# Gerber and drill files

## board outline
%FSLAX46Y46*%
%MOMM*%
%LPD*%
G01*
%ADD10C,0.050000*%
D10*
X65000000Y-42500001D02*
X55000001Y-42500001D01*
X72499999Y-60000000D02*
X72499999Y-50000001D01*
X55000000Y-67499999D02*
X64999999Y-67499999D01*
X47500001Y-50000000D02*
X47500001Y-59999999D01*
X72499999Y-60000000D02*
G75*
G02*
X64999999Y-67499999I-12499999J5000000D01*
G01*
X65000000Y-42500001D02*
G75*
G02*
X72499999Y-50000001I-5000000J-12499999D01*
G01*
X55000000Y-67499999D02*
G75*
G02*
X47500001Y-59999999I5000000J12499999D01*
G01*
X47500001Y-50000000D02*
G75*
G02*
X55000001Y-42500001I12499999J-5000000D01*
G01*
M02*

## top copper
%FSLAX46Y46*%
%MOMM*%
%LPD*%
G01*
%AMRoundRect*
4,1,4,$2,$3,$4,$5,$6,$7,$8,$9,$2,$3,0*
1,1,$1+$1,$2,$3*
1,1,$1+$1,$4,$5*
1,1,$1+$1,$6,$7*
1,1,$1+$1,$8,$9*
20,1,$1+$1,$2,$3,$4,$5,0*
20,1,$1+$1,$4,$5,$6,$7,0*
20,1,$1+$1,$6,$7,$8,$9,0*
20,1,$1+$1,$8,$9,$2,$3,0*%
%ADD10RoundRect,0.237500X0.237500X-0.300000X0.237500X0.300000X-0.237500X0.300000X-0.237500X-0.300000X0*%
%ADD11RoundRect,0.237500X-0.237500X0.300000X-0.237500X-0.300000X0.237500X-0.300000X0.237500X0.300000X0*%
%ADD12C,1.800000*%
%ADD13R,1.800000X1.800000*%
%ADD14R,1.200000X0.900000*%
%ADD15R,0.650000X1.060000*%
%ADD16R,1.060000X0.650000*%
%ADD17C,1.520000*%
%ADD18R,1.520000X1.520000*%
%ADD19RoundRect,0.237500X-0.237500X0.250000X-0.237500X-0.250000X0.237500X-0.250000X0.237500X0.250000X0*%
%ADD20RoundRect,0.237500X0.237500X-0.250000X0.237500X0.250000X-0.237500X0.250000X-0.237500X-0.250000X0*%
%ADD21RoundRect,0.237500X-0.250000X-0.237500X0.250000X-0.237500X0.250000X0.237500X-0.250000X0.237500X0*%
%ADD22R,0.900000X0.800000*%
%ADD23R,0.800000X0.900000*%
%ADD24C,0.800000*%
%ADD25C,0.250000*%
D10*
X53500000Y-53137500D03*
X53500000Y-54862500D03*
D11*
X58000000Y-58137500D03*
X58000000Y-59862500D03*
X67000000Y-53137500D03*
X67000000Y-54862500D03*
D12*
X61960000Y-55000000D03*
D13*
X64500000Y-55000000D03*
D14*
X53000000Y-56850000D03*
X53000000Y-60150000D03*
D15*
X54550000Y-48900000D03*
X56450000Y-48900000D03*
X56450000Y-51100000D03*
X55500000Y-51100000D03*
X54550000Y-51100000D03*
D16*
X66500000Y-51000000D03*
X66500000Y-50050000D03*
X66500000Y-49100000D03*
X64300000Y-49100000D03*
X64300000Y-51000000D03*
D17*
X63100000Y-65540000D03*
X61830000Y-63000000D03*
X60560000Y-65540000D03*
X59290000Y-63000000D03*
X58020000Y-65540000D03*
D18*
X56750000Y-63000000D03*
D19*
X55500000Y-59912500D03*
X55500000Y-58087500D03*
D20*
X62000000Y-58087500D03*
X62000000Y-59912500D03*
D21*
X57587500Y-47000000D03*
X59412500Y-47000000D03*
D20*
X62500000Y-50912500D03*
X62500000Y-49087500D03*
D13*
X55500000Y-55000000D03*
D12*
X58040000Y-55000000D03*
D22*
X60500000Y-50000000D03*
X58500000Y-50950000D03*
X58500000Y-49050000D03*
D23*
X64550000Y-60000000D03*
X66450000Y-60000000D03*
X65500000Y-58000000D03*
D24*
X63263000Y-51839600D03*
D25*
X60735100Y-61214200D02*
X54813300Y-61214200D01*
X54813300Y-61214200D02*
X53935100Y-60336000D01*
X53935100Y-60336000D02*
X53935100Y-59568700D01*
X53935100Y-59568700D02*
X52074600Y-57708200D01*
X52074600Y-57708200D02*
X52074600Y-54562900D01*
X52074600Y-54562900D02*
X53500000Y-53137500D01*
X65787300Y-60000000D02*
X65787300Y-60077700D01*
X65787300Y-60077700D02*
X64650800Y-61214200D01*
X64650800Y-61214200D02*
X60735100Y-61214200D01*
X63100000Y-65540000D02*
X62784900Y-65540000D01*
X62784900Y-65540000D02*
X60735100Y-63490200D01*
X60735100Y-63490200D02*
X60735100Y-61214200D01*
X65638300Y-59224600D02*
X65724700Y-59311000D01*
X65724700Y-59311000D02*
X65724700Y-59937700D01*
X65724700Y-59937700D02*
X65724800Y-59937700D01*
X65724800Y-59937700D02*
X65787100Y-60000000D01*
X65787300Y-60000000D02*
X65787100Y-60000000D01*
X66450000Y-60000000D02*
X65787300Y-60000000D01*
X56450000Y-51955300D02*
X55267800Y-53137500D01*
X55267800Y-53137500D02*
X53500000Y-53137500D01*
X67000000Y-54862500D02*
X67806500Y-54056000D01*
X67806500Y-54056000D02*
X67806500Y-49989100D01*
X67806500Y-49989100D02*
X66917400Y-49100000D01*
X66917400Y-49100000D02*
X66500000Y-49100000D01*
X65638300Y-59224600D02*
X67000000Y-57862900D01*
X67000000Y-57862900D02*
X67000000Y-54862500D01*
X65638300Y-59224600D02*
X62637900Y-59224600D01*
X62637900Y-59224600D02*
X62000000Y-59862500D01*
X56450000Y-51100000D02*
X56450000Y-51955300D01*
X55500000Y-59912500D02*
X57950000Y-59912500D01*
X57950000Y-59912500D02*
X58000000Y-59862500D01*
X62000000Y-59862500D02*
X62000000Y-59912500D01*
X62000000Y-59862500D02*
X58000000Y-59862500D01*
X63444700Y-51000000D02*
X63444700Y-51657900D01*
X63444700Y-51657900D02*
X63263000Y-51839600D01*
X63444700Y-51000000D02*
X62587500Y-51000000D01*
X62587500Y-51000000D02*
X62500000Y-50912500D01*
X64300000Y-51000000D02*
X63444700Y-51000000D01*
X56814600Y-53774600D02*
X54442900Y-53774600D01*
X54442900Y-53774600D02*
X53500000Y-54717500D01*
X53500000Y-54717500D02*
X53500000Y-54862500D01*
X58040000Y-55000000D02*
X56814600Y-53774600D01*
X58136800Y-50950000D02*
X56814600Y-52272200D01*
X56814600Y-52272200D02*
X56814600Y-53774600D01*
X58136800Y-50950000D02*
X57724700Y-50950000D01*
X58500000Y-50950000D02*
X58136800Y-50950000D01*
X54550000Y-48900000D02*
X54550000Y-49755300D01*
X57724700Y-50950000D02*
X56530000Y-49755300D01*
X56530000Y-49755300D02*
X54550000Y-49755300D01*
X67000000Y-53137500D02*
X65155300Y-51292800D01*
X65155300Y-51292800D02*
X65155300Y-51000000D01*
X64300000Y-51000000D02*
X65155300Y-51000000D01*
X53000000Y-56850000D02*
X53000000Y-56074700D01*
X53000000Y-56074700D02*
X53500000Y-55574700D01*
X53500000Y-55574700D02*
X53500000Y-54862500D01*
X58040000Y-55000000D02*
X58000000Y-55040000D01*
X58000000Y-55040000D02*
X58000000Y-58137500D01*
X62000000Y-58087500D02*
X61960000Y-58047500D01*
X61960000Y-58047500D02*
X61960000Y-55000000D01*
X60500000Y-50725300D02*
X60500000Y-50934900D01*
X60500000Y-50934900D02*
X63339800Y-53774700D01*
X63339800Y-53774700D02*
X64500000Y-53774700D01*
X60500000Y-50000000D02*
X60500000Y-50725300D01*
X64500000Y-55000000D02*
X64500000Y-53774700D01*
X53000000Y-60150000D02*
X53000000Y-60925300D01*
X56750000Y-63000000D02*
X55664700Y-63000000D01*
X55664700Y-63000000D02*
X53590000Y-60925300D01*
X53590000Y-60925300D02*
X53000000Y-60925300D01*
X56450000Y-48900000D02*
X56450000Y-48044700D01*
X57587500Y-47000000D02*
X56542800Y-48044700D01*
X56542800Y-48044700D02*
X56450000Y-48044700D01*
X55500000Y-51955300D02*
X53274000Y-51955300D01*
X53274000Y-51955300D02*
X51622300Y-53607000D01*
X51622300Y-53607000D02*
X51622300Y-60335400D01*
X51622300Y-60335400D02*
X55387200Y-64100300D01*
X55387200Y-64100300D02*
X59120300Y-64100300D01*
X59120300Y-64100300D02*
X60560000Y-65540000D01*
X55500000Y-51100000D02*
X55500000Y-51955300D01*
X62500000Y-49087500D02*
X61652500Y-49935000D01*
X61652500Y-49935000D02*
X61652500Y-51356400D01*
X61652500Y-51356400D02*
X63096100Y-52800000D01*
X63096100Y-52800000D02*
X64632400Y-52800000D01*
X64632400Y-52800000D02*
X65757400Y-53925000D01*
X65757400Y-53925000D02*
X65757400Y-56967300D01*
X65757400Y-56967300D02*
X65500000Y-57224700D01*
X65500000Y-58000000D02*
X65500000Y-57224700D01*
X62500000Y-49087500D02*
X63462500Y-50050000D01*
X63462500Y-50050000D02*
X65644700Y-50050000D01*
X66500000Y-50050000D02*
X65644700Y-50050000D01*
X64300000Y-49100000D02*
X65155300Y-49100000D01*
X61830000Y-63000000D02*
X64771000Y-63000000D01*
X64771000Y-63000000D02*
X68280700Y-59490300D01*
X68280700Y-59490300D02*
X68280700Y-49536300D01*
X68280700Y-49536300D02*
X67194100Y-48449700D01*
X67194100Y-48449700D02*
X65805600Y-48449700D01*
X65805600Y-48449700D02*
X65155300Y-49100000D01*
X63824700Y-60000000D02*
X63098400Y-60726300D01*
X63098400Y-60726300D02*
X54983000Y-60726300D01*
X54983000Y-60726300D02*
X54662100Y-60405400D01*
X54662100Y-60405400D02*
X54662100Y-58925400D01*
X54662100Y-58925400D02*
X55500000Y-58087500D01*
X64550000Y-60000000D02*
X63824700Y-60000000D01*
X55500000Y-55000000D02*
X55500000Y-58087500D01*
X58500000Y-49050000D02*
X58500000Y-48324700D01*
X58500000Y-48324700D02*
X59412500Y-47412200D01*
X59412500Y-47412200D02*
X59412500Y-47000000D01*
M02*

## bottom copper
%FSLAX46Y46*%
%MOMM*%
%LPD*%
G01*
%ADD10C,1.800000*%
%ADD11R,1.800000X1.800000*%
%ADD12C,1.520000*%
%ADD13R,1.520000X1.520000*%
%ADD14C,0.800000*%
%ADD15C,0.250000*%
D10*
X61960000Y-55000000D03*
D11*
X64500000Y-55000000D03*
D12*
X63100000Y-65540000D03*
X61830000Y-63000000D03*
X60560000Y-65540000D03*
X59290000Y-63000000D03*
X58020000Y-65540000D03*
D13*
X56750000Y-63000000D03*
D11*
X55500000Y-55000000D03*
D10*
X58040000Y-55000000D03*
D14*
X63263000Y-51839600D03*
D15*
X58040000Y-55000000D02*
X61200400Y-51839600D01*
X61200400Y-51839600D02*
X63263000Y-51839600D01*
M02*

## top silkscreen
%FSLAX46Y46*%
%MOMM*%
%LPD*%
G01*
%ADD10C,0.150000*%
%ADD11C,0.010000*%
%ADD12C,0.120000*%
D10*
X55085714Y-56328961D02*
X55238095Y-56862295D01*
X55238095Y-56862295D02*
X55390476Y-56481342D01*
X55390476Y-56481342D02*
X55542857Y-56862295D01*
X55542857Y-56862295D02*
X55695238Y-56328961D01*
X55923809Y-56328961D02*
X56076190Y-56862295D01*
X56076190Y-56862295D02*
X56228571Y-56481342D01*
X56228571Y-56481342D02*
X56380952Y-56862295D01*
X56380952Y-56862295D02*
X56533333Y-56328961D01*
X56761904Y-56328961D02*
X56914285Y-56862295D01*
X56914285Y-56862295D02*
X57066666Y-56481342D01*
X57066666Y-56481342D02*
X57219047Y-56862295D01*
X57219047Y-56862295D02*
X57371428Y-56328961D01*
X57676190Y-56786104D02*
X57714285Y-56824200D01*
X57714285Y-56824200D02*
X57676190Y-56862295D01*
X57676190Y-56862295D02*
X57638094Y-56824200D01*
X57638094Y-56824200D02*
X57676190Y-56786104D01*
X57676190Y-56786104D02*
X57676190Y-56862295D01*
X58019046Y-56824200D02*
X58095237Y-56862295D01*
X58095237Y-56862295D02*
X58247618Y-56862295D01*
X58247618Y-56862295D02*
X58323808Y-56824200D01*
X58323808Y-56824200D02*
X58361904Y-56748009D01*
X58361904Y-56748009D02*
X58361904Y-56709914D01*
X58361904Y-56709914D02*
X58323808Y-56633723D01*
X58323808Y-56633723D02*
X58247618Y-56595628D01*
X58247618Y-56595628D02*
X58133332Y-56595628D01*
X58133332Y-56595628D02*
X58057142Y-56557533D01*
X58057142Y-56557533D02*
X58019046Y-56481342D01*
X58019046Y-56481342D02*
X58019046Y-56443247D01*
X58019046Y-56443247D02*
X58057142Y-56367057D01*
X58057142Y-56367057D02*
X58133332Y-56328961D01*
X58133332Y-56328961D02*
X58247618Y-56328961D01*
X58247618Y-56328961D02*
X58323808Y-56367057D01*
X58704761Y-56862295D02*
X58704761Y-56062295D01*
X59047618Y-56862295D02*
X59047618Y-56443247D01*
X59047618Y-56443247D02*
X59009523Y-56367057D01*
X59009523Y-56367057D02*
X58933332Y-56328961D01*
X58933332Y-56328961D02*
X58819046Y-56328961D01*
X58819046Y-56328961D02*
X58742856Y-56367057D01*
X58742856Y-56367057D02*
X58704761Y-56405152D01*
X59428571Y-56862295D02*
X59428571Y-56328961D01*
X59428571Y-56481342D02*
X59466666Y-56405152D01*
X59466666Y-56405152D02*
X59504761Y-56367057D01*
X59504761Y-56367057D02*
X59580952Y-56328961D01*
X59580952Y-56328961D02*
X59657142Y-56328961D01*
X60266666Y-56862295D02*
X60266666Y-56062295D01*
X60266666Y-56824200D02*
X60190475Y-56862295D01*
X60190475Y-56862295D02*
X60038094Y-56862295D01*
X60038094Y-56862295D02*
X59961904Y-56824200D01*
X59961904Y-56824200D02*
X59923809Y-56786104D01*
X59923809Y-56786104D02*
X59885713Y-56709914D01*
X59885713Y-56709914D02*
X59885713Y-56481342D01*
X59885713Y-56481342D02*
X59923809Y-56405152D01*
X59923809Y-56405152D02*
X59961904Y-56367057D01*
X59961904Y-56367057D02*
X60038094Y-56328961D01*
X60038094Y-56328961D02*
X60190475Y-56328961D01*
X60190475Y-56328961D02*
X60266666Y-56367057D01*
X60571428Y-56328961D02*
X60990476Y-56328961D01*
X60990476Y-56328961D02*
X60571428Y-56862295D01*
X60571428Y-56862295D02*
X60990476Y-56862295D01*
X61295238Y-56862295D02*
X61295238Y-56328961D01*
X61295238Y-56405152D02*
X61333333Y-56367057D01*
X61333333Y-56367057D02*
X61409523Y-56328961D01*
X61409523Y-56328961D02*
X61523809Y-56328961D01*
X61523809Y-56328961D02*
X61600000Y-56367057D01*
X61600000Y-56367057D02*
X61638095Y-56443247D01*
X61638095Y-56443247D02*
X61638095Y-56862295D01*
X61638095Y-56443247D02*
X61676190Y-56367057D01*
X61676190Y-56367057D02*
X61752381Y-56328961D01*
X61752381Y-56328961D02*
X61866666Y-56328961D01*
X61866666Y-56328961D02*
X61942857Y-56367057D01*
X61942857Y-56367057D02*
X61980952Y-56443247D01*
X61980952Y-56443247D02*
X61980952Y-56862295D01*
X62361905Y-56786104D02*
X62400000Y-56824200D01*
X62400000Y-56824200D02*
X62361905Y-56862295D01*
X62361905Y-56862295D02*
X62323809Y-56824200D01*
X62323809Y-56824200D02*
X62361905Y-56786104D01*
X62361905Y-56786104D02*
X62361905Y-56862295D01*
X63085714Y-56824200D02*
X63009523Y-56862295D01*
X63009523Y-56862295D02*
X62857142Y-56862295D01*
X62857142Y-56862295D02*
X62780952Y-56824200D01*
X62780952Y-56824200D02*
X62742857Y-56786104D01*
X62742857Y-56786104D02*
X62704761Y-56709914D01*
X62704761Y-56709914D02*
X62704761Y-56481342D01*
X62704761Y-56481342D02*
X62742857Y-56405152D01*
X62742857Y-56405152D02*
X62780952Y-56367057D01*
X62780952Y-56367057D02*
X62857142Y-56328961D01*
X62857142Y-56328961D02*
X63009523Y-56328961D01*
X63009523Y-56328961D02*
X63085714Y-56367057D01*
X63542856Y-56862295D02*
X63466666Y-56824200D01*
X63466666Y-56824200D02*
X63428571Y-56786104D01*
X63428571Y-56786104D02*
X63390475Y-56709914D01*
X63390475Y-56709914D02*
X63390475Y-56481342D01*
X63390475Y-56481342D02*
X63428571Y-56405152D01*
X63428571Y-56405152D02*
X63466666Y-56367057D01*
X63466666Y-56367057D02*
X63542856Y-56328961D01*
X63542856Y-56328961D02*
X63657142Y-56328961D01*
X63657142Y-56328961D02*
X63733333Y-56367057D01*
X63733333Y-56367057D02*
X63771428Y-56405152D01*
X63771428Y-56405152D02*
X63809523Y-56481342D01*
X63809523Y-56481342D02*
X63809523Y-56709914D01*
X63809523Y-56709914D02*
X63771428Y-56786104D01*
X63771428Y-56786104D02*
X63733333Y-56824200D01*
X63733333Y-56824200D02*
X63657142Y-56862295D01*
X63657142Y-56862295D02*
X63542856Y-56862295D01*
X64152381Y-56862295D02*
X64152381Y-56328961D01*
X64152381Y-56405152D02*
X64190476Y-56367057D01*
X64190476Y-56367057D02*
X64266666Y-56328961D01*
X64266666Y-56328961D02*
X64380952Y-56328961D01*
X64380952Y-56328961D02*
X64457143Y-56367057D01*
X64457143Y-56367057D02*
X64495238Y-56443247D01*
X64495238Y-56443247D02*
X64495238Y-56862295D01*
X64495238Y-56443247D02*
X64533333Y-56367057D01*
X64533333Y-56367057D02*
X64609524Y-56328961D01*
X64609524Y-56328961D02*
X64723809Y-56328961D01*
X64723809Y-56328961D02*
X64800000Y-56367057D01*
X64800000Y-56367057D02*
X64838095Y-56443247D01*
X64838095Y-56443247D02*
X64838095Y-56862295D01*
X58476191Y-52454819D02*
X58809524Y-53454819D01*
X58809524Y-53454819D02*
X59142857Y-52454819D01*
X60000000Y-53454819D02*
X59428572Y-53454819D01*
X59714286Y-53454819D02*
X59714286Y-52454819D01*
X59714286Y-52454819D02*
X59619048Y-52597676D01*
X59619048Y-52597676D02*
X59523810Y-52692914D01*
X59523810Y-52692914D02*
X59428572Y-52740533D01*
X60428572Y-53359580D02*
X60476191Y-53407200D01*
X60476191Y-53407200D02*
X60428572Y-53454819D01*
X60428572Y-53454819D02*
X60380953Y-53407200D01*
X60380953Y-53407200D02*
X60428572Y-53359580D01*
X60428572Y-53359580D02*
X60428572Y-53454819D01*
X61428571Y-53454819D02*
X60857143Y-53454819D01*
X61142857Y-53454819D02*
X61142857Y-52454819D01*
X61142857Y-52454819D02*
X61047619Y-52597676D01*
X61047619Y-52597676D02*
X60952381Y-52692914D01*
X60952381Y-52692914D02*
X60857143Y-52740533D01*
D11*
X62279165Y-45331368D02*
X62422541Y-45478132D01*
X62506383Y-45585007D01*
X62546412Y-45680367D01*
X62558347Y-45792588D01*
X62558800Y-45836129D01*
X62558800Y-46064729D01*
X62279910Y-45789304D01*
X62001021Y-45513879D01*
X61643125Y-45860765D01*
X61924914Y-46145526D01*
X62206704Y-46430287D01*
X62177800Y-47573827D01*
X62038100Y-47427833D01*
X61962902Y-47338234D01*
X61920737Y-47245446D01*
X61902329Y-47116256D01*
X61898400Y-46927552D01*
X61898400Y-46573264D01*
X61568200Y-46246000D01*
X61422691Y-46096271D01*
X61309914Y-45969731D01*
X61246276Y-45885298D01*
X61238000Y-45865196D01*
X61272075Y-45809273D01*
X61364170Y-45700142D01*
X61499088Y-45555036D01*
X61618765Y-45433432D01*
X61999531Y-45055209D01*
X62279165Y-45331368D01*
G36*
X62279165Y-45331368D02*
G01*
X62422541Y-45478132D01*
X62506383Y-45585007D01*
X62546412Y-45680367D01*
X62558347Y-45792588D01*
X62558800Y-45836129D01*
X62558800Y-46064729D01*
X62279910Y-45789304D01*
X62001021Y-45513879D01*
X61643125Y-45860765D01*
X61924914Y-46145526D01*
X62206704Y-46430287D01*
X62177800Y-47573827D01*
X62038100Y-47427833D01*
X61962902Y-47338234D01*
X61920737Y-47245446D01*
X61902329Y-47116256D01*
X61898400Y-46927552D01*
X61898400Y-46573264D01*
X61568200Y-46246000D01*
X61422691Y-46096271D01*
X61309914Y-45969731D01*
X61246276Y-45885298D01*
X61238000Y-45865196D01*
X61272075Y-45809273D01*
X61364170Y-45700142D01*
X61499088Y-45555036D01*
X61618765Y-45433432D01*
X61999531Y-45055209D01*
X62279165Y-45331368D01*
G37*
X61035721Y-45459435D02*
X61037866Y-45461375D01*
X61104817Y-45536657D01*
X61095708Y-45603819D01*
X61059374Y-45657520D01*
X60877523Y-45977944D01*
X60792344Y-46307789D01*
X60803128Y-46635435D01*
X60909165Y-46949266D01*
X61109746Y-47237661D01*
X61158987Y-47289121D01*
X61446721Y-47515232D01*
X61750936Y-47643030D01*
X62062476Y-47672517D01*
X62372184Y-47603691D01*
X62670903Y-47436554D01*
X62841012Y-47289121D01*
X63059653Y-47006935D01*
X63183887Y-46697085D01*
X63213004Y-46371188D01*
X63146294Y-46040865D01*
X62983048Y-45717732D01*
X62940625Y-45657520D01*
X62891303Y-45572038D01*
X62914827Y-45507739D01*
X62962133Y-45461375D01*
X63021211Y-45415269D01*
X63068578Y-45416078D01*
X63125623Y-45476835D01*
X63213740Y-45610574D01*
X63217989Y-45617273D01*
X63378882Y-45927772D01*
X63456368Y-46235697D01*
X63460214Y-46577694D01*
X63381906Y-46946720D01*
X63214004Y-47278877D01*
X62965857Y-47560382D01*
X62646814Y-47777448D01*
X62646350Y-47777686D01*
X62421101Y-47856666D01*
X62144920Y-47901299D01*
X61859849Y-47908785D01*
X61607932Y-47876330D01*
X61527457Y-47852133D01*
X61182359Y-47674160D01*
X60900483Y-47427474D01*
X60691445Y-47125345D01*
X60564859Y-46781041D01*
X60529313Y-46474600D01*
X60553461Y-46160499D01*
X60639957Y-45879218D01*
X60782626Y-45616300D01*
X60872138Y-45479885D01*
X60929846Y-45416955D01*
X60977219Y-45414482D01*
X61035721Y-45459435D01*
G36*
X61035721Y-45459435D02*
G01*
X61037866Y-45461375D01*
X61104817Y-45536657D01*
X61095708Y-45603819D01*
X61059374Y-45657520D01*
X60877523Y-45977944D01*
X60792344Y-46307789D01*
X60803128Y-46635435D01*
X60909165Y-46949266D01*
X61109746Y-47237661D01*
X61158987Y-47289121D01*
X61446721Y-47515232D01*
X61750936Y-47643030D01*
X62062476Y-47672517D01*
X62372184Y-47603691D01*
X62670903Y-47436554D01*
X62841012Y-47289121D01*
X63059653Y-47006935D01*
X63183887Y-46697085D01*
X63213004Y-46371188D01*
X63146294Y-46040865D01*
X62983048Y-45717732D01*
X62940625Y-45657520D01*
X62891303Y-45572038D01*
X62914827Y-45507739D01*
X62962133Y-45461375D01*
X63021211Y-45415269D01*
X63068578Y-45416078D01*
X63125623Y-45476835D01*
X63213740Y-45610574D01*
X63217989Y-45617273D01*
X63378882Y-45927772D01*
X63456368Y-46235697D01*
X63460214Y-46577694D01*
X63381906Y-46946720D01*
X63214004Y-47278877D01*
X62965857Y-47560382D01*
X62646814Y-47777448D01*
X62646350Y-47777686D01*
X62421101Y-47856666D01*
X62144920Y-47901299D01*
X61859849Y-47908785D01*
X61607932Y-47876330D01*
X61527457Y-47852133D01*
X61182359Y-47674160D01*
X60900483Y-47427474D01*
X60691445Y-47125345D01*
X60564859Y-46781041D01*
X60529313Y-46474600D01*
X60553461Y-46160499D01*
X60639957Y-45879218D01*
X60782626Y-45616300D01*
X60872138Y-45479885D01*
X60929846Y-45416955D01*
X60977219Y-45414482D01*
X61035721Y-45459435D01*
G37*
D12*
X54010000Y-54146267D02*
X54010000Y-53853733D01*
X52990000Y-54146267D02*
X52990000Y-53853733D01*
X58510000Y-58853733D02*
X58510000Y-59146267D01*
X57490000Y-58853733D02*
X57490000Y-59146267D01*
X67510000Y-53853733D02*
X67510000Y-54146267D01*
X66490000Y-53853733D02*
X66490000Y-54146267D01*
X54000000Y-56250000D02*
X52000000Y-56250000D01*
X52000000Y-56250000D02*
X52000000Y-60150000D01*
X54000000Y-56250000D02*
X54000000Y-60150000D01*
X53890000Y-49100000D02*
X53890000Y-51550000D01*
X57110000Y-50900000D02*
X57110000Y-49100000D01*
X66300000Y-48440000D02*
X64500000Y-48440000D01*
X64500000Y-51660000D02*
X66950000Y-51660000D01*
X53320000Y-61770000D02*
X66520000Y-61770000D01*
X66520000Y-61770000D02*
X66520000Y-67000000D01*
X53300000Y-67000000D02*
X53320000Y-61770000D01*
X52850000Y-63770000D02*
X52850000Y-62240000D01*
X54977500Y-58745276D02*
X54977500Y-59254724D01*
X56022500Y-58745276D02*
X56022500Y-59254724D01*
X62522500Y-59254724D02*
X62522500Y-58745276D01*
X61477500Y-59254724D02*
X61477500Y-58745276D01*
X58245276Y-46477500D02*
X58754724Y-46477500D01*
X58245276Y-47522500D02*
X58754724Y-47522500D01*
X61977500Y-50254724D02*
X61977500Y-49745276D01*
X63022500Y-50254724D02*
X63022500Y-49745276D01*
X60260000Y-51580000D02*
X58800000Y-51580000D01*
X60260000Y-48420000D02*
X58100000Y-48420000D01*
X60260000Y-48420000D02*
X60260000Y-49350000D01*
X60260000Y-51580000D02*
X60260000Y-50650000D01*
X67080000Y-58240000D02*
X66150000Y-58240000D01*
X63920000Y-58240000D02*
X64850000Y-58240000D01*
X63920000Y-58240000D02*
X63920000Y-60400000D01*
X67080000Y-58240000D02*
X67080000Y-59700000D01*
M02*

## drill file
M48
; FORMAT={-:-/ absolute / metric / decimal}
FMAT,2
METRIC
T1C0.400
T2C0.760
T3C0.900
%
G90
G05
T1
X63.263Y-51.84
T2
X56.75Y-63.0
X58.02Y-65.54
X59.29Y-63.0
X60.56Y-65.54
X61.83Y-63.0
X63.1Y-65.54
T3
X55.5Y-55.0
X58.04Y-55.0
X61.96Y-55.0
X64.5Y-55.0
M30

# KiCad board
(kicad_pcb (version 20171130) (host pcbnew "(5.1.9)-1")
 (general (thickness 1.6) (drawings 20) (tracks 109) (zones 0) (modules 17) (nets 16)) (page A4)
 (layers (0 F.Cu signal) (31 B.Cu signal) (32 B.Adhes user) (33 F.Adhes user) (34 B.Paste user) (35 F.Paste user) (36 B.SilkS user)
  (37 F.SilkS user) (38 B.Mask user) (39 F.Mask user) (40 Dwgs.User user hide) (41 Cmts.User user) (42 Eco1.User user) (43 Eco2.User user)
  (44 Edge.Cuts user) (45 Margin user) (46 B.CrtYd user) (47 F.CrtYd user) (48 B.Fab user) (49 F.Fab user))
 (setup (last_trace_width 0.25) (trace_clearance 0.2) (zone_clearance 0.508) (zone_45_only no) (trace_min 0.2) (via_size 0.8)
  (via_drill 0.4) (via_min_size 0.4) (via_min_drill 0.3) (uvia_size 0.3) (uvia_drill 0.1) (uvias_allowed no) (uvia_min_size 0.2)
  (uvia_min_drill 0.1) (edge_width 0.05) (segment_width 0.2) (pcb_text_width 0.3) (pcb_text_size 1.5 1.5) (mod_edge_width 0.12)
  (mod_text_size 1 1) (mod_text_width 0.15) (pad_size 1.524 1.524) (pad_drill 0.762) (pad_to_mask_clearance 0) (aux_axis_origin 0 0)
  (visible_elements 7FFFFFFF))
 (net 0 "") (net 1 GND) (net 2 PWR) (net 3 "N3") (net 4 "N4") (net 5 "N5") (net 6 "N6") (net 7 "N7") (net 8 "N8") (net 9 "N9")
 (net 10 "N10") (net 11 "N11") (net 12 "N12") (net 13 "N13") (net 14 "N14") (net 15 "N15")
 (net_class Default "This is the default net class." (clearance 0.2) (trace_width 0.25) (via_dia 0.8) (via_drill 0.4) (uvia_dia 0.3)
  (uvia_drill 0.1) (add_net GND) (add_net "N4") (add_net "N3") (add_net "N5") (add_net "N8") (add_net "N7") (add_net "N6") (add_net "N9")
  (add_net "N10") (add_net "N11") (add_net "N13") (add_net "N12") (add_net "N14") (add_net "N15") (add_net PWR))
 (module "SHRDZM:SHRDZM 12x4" (layer B.Cu) (at 60.5 50 180)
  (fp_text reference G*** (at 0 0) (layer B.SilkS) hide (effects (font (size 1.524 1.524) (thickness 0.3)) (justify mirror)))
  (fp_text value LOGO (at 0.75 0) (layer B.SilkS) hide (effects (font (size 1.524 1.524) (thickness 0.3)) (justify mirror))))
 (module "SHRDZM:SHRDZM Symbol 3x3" (layer F.Cu) (at 62 46.5)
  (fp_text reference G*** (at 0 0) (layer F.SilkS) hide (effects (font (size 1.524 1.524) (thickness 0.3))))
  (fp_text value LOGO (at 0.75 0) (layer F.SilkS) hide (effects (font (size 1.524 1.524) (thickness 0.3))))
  (fp_poly
   (pts (xy 0.279165 -1.168632) (xy 0.422541 -1.021868) (xy 0.506383 -0.914993) (xy 0.546412 -0.819633) (xy 0.558347 -0.707412)
    (xy 0.5588 -0.663871) (xy 0.5588 -0.435271) (xy 0.27991 -0.710696) (xy 0.001021 -0.986121) (xy -0.356875 -0.639235)
    (xy -0.075086 -0.354474) (xy 0.206704 -0.069713) (xy 0.1778 1.073827) (xy 0.0381 0.927833) (xy -0.037098 0.838234)
    (xy -0.079263 0.745446) (xy -0.097671 0.616256) (xy -0.1016 0.427552) (xy -0.1016 0.073264) (xy -0.4318 -0.254) (xy -0.577309 -0.403729)
    (xy -0.690086 -0.530269) (xy -0.753724 -0.614702) (xy -0.762 -0.634804) (xy -0.727925 -0.690727) (xy -0.63583 -0.799858)
    (xy -0.500912 -0.944964) (xy -0.381235 -1.066568) (xy -0.000469 -1.444791) (xy 0.279165 -1.168632))
   (layer F.SilkS) (width 0.01))
  (fp_poly
   (pts (xy -0.964279 -1.040565) (xy -0.962134 -1.038625) (xy -0.895183 -0.963343) (xy -0.904292 -0.896181) (xy -0.940626 -0.84248)
    (xy -1.122477 -0.522056) (xy -1.207656 -0.192211) (xy -1.196872 0.135435) (xy -1.090835 0.449266) (xy -0.890254 0.737661)
    (xy -0.841013 0.789121) (xy -0.553279 1.015232) (xy -0.249064 1.14303) (xy 0.062476 1.172517) (xy 0.372184 1.103691)
    (xy 0.670903 0.936554) (xy 0.841012 0.789121) (xy 1.059653 0.506935) (xy 1.183887 0.197085) (xy 1.213004 -0.128812)
    (xy 1.146294 -0.459135) (xy 0.983048 -0.782268) (xy 0.940625 -0.84248) (xy 0.891303 -0.927962) (xy 0.914827 -0.992261)
    (xy 0.962133 -1.038625) (xy 1.021211 -1.084731) (xy 1.068578 -1.083922) (xy 1.125623 -1.023165) (xy 1.21374 -0.889426)
    (xy 1.217989 -0.882727) (xy 1.378882 -0.572228) (xy 1.456368 -0.264303) (xy 1.460214 0.077694) (xy 1.381906 0.44672)
    (xy 1.214004 0.778877) (xy 0.965857 1.060382) (xy 0.646814 1.277448) (xy 0.64635 1.277686) (xy 0.421101 1.356666) (xy 0.14492 1.401299)
    (xy -0.140151 1.408785) (xy -0.392068 1.37633) (xy -0.472543 1.352133) (xy -0.817641 1.17416) (xy -1.099517 0.927474)
    (xy -1.308555 0.625345) (xy -1.435141 0.281041) (xy -1.470687 -0.0254) (xy -1.446539 -0.339501) (xy -1.360043 -0.620782)
    (xy -1.217374 -0.8837) (xy -1.127862 -1.020115) (xy -1.070154 -1.083045) (xy -1.022781 -1.085518) (xy -0.964279 -1.040565))
   (layer F.SilkS) (width 0.01)))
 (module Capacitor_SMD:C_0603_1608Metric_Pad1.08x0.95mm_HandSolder (layer F.Cu) (at 53.5 54 90)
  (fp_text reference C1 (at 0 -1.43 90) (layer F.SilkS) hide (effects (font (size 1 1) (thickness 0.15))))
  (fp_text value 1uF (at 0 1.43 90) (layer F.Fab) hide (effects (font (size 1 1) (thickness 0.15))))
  (fp_line (start -0.146267 0.51) (end 0.146267 0.51) (layer F.SilkS) (width 0.12))
  (fp_line (start -0.146267 -0.51) (end 0.146267 -0.51) (layer F.SilkS) (width 0.12))
  (pad 2 smd roundrect (at 0.8625 0 90) (size 1.075 0.95) (layers F.Cu F.Paste F.Mask) (roundrect_rratio 0.25) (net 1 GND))
  (pad 1 smd roundrect (at -0.8625 0 90) (size 1.075 0.95) (layers F.Cu F.Paste F.Mask) (roundrect_rratio 0.25) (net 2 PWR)))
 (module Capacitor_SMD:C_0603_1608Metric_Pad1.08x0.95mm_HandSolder (layer F.Cu) (at 58 59 270)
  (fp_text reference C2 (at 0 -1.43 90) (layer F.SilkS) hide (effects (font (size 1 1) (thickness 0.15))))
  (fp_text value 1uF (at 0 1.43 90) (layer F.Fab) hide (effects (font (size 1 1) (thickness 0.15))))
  (fp_line (start -0.146267 -0.51) (end 0.146267 -0.51) (layer F.SilkS) (width 0.12))
  (fp_line (start -0.146267 0.51) (end 0.146267 0.51) (layer F.SilkS) (width 0.12))
  (pad 1 smd roundrect (at -0.8625 0 270) (size 1.075 0.95) (layers F.Cu F.Paste F.Mask) (roundrect_rratio 0.25) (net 2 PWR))
  (pad 2 smd roundrect (at 0.8625 0 270) (size 1.075 0.95) (layers F.Cu F.Paste F.Mask) (roundrect_rratio 0.25) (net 1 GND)))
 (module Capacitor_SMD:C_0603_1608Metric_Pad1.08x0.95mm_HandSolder (layer F.Cu) (at 67 54 270)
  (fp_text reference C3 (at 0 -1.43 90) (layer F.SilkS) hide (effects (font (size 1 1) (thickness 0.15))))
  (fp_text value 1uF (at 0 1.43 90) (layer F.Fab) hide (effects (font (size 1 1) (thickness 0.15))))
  (fp_line (start -0.146267 -0.51) (end 0.146267 -0.51) (layer F.SilkS) (width 0.12))
  (fp_line (start -0.146267 0.51) (end 0.146267 0.51) (layer F.SilkS) (width 0.12))
  (pad 1 smd roundrect (at -0.8625 0 270) (size 1.075 0.95) (layers F.Cu F.Paste F.Mask) (roundrect_rratio 0.25) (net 2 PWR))
  (pad 2 smd roundrect (at 0.8625 0 270) (size 1.075 0.95) (layers F.Cu F.Paste F.Mask) (roundrect_rratio 0.25) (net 1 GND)))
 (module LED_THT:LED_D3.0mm (layer B.Cu) (at 64.5 55 180)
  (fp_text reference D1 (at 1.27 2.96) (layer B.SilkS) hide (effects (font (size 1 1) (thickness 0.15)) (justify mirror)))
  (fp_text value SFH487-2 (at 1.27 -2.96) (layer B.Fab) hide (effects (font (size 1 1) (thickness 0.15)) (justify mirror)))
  (pad 2 thru_hole circle (at 2.54 0 180) (size 1.8 1.8) (drill 0.9) (layers *.Cu *.Mask) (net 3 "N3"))
  (pad 1 thru_hole rect (at 0 0 180) (size 1.8 1.8) (drill 0.9) (layers *.Cu *.Mask) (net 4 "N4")))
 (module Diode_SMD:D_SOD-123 (layer F.Cu) (at 53 58.5 270)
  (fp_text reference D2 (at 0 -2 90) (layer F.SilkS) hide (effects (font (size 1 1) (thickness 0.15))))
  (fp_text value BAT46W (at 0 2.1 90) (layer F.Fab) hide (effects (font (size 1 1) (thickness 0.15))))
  (fp_line (start -2.25 -1) (end -2.25 1) (layer F.SilkS) (width 0.12))
  (fp_line (start -2.25 1) (end 1.65 1) (layer F.SilkS) (width 0.12))
  (fp_line (start -2.25 -1) (end 1.65 -1) (layer F.SilkS) (width 0.12))
  (pad 1 smd rect (at -1.65 0 270) (size 0.9 1.2) (layers F.Cu F.Paste F.Mask) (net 2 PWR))
  (pad 2 smd rect (at 1.65 0 270) (size 0.9 1.2) (layers F.Cu F.Paste F.Mask) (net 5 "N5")))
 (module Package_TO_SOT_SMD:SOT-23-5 (layer F.Cu) (at 55.5 50 90)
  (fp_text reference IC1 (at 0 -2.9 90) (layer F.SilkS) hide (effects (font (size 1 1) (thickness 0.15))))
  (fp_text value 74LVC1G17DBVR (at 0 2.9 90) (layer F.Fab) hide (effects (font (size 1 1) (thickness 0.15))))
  (fp_line (start 0.9 -1.61) (end -1.55 -1.61) (layer F.SilkS) (width 0.12))
  (fp_line (start -0.9 1.61) (end 0.9 1.61) (layer F.SilkS) (width 0.12))
  (pad 5 smd rect (at 1.1 -0.95 90) (size 1.06 0.65) (layers F.Cu F.Paste F.Mask) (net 2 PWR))
  (pad 4 smd rect (at 1.1 0.95 90) (size 1.06 0.65) (layers F.Cu F.Paste F.Mask) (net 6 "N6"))
  (pad 3 smd rect (at -1.1 0.95 90) (size 1.06 0.65) (layers F.Cu F.Paste F.Mask) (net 1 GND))
  (pad 2 smd rect (at -1.1 0 90) (size 1.06 0.65) (layers F.Cu F.Paste F.Mask) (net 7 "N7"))
  (pad 1 smd rect (at -1.1 -0.95 90) (size 1.06 0.65) (layers F.Cu F.Paste F.Mask) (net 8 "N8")))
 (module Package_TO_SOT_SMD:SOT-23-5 (layer F.Cu) (at 65.4 50.05 180)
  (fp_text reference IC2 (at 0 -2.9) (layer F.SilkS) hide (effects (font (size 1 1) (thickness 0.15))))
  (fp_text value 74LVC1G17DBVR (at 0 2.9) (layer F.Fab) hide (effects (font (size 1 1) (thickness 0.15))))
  (fp_line (start -0.9 1.61) (end 0.9 1.61) (layer F.SilkS) (width 0.12))
  (fp_line (start 0.9 -1.61) (end -1.55 -1.61) (layer F.SilkS) (width 0.12))
  (pad 1 smd rect (at -1.1 -0.95 180) (size 1.06 0.65) (layers F.Cu F.Paste F.Mask) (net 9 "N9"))
  (pad 2 smd rect (at -1.1 0 180) (size 1.06 0.65) (layers F.Cu F.Paste F.Mask) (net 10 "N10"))
  (pad 3 smd rect (at -1.1 0.95 180) (size 1.06 0.65) (layers F.Cu F.Paste F.Mask) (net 1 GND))
  (pad 4 smd rect (at 1.1 0.95 180) (size 1.06 0.65) (layers F.Cu F.Paste F.Mask) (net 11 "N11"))
  (pad 5 smd rect (at 1.1 -0.95 180) (size 1.06 0.65) (layers F.Cu F.Paste F.Mask) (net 2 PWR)))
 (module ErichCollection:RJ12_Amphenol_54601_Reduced (layer F.Cu) (at 56.75 63)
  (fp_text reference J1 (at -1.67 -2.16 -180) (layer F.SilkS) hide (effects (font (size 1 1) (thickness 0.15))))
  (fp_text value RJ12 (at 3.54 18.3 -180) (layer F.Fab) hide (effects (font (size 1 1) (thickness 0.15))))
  (fp_line (start -3.43 -1.23) (end 9.77 -1.23) (layer F.SilkS) (width 0.12))
  (fp_line (start 9.77 -1.23) (end 9.77 4) (layer F.SilkS) (width 0.12))
  (fp_line (start -3.45 4) (end -3.43 -1.23) (layer F.SilkS) (width 0.12))
  (fp_line (start -3.9 0.77) (end -3.9 -0.76) (layer F.SilkS) (width 0.12))
  (pad 6 thru_hole circle (at 6.35 2.54) (size 1.52 1.52) (drill 0.76) (layers *.Cu *.Mask) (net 1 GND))
  (pad 5 thru_hole circle (at 5.08 0) (size 1.52 1.52) (drill 0.76) (layers *.Cu *.Mask) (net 11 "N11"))
  (pad 4 thru_hole circle (at 3.81 2.54) (size 1.52 1.52) (drill 0.76) (layers *.Cu *.Mask) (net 7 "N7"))
  (pad 3 thru_hole circle (at 2.54 0) (size 1.52 1.52) (drill 0.76) (layers *.Cu *.Mask) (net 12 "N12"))
  (pad 2 thru_hole circle (at 1.27 2.54) (size 1.52 1.52) (drill 0.76) (layers *.Cu *.Mask) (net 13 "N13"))
  (pad 1 thru_hole rect (at 0 0) (size 1.52 1.52) (drill 0.76) (layers *.Cu *.Mask) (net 5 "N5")))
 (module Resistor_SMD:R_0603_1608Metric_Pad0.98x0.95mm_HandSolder (layer F.Cu) (at 55.5 59 270)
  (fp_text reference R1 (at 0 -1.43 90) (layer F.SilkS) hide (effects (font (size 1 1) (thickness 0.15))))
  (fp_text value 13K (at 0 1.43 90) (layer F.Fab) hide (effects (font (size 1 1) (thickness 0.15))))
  (fp_line (start -0.254724 0.5225) (end 0.254724 0.5225) (layer F.SilkS) (width 0.12))
  (fp_line (start -0.254724 -0.5225) (end 0.254724 -0.5225) (layer F.SilkS) (width 0.12))
  (pad 2 smd roundrect (at 0.9125 0 270) (size 0.975 0.95) (layers F.Cu F.Paste F.Mask) (roundrect_rratio 0.25) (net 1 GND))
  (pad 1 smd roundrect (at -0.9125 0 270) (size 0.975 0.95) (layers F.Cu F.Paste F.Mask) (roundrect_rratio 0.25) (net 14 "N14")))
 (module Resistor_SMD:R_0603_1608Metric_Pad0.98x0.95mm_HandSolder (layer F.Cu) (at 62 59 90)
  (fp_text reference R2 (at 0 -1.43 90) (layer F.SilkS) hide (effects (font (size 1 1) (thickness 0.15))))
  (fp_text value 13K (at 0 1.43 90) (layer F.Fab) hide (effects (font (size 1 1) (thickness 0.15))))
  (fp_line (start -0.254724 0.5225) (end 0.254724 0.5225) (layer F.SilkS) (width 0.12))
  (fp_line (start -0.254724 -0.5225) (end 0.254724 -0.5225) (layer F.SilkS) (width 0.12))
  (pad 2 smd roundrect (at 0.9125 0 90) (size 0.975 0.95) (layers F.Cu F.Paste F.Mask) (roundrect_rratio 0.25) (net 3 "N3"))
  (pad 1 smd roundrect (at -0.9125 0 90) (size 0.975 0.95) (layers F.Cu F.Paste F.Mask) (roundrect_rratio 0.25) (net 1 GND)))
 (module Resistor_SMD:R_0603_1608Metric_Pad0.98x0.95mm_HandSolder (layer F.Cu) (at 58.5 47)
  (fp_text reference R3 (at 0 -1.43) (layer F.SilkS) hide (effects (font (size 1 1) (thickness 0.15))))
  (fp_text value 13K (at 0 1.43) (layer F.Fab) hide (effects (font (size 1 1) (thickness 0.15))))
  (fp_line (start -0.254724 -0.5225) (end 0.254724 -0.5225) (layer F.SilkS) (width 0.12))
  (fp_line (start -0.254724 0.5225) (end 0.254724 0.5225) (layer F.SilkS) (width 0.12))
  (pad 1 smd roundrect (at -0.9125 0) (size 0.975 0.95) (layers F.Cu F.Paste F.Mask) (roundrect_rratio 0.25) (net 6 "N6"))
  (pad 2 smd roundrect (at 0.9125 0) (size 0.975 0.95) (layers F.Cu F.Paste F.Mask) (roundrect_rratio 0.25) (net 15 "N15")))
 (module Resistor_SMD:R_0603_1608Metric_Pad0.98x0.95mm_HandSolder (layer F.Cu) (at 62.5 50 90)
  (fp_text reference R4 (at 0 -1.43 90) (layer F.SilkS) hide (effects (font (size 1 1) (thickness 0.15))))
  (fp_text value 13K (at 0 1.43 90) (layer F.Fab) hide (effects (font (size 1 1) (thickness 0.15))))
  (fp_line (start -0.254724 -0.5225) (end 0.254724 -0.5225) (layer F.SilkS) (width 0.12))
  (fp_line (start -0.254724 0.5225) (end 0.254724 0.5225) (layer F.SilkS) (width 0.12))
  (pad 1 smd roundrect (at -0.9125 0 90) (size 0.975 0.95) (layers F.Cu F.Paste F.Mask) (roundrect_rratio 0.25) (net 2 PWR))
  (pad 2 smd roundrect (at 0.9125 0 90) (size 0.975 0.95) (layers F.Cu F.Paste F.Mask) (roundrect_rratio 0.25) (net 10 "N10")))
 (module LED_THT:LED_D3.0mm (layer B.Cu) (at 55.5 55)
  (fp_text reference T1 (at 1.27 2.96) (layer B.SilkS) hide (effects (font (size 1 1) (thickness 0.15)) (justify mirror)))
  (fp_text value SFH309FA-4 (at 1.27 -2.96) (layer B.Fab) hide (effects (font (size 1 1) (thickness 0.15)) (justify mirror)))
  (pad 1 thru_hole rect (at 0 0) (size 1.8 1.8) (drill 0.9) (layers *.Cu *.Mask) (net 14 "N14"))
  (pad 2 thru_hole circle (at 2.54 0) (size 1.8 1.8) (drill 0.9) (layers *.Cu *.Mask) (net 2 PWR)))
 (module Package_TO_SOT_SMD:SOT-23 (layer F.Cu) (at 59.5 50)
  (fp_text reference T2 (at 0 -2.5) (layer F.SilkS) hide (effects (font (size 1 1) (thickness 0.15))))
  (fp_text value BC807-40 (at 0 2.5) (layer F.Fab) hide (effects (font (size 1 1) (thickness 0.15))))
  (fp_line (start 0.76 1.58) (end -0.7 1.58) (layer F.SilkS) (width 0.12))
  (fp_line (start 0.76 -1.58) (end -1.4 -1.58) (layer F.SilkS) (width 0.12))
  (fp_line (start 0.76 -1.58) (end 0.76 -0.65) (layer F.SilkS) (width 0.12))
  (fp_line (start 0.76 1.58) (end 0.76 0.65) (layer F.SilkS) (width 0.12))
  (pad 3 smd rect (at 1 0) (size 0.9 0.8) (layers F.Cu F.Paste F.Mask) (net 4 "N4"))
  (pad 2 smd rect (at -1 0.95) (size 0.9 0.8) (layers F.Cu F.Paste F.Mask) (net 2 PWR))
  (pad 1 smd rect (at -1 -0.95) (size 0.9 0.8) (layers F.Cu F.Paste F.Mask) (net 15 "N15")))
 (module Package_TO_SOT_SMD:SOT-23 (layer F.Cu) (at 65.5 59 90)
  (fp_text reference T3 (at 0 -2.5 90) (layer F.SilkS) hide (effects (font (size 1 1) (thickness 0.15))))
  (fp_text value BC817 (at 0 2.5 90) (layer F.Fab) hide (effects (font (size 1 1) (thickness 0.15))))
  (fp_line (start 0.76 1.58) (end 0.76 0.65) (layer F.SilkS) (width 0.12))
  (fp_line (start 0.76 -1.58) (end 0.76 -0.65) (layer F.SilkS) (width 0.12))
  (fp_line (start 0.76 -1.58) (end -1.4 -1.58) (layer F.SilkS) (width 0.12))
  (fp_line (start 0.76 1.58) (end -0.7 1.58) (layer F.SilkS) (width 0.12))
  (pad 1 smd rect (at -1 -0.95 90) (size 0.9 0.8) (layers F.Cu F.Paste F.Mask) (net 14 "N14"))
  (pad 2 smd rect (at -1 0.95 90) (size 0.9 0.8) (layers F.Cu F.Paste F.Mask) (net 1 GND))
  (pad 3 smd rect (at 1 0 90) (size 0.9 0.8) (layers F.Cu F.Paste F.Mask) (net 10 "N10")))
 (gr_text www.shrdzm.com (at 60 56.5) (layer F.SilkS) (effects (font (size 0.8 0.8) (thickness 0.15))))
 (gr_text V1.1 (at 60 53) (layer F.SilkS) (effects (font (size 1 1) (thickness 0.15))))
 (gr_line (start 65 42.500001) (end 55.000001 42.500001) (layer Edge.Cuts) (width 0.05))
 (gr_line (start 72.499999 60) (end 72.499999 50.000001) (layer Edge.Cuts) (width 0.05))
 (gr_line (start 55 67.499999) (end 64.999999 67.499999) (layer Edge.Cuts) (width 0.05))
 (gr_line (start 47.500001 50) (end 47.500001 59.999999) (layer Edge.Cuts) (width 0.05))
 (gr_arc (start 60 55) (end 64.999999 67.499999) (angle -46.39718103) (layer Edge.Cuts) (width 0.05))
 (gr_arc (start 60 55) (end 72.499999 50.000001) (angle -46.39718103) (layer Edge.Cuts) (width 0.05))
 (gr_arc (start 60 55) (end 47.500001 59.999999) (angle -46.39718103) (layer Edge.Cuts) (width 0.05))
 (gr_arc (start 60 55) (end 55.000001 42.500001) (angle -46.39718103) (layer Edge.Cuts) (width 0.05))
 (segment (start 60.7351 61.2142) (end 54.8133 61.2142) (width 0.25) (layer F.Cu) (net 1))
 (segment (start 54.8133 61.2142) (end 53.9351 60.336) (width 0.25) (layer F.Cu) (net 1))
 (segment (start 53.9351 60.336) (end 53.9351 59.5687) (width 0.25) (layer F.Cu) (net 1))
 (segment (start 53.9351 59.5687) (end 52.0746 57.7082) (width 0.25) (layer F.Cu) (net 1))
 (segment (start 52.0746 57.7082) (end 52.0746 54.5629) (width 0.25) (layer F.Cu) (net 1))
 (segment (start 52.0746 54.5629) (end 53.5 53.1375) (width 0.25) (layer F.Cu) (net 1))
 (segment (start 65.7873 60) (end 65.7873 60.0777) (width 0.25) (layer F.Cu) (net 1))
 (segment (start 65.7873 60.0777) (end 64.6508 61.2142) (width 0.25) (layer F.Cu) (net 1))
 (segment (start 64.6508 61.2142) (end 60.7351 61.2142) (width 0.25) (layer F.Cu) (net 1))
 (segment (start 63.1 65.54) (end 62.7849 65.54) (width 0.25) (layer F.Cu) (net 1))
 (segment (start 62.7849 65.54) (end 60.7351 63.4902) (width 0.25) (layer F.Cu) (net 1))
 (segment (start 60.7351 63.4902) (end 60.7351 61.2142) (width 0.25) (layer F.Cu) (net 1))
 (segment (start 65.6383 59.2246) (end 65.7247 59.311) (width 0.25) (layer F.Cu) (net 1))
 (segment (start 65.7247 59.311) (end 65.7247 59.9377) (width 0.25) (layer F.Cu) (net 1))
 (segment (start 65.7247 59.9377) (end 65.7248 59.9377) (width 0.25) (layer F.Cu) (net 1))
 (segment (start 65.7248 59.9377) (end 65.7871 60) (width 0.25) (layer F.Cu) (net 1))
 (segment (start 65.7873 60) (end 65.7871 60) (width 0.25) (layer F.Cu) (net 1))
 (segment (start 66.45 60) (end 65.7873 60) (width 0.25) (layer F.Cu) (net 1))
 (segment (start 56.45 51.9553) (end 55.2678 53.1375) (width 0.25) (layer F.Cu) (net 1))
 (segment (start 55.2678 53.1375) (end 53.5 53.1375) (width 0.25) (layer F.Cu) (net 1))
 (segment (start 67 54.8625) (end 67.8065 54.056) (width 0.25) (layer F.Cu) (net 1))
 (segment (start 67.8065 54.056) (end 67.8065 49.9891) (width 0.25) (layer F.Cu) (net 1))
 (segment (start 67.8065 49.9891) (end 66.9174 49.1) (width 0.25) (layer F.Cu) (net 1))
 (segment (start 66.9174 49.1) (end 66.5 49.1) (width 0.25) (layer F.Cu) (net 1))
 (segment (start 65.6383 59.2246) (end 67 57.8629) (width 0.25) (layer F.Cu) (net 1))
 (segment (start 67 57.8629) (end 67 54.8625) (width 0.25) (layer F.Cu) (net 1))
 (segment (start 65.6383 59.2246) (end 62.6379 59.2246) (width 0.25) (layer F.Cu) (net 1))
 (segment (start 62.6379 59.2246) (end 62 59.8625) (width 0.25) (layer F.Cu) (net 1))
 (segment (start 56.45 51.1) (end 56.45 51.9553) (width 0.25) (layer F.Cu) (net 1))
 (segment (start 55.5 59.9125) (end 57.95 59.9125) (width 0.25) (layer F.Cu) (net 1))
 (segment (start 57.95 59.9125) (end 58 59.8625) (width 0.25) (layer F.Cu) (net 1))
 (segment (start 62 59.8625) (end 62 59.9125) (width 0.25) (layer F.Cu) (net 1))
 (segment (start 62 59.8625) (end 58 59.8625) (width 0.25) (layer F.Cu) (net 1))
 (segment (start 63.4447 51) (end 63.4447 51.6579) (width 0.25) (layer F.Cu) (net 2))
 (segment (start 63.4447 51.6579) (end 63.263 51.8396) (width 0.25) (layer F.Cu) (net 2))
 (segment (start 58.04 55) (end 61.2004 51.8396) (width 0.25) (layer B.Cu) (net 2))
 (segment (start 61.2004 51.8396) (end 63.263 51.8396) (width 0.25) (layer B.Cu) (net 2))
 (segment (start 63.4447 51) (end 62.5875 51) (width 0.25) (layer F.Cu) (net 2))
 (segment (start 62.5875 51) (end 62.5 50.9125) (width 0.25) (layer F.Cu) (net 2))
 (segment (start 64.3 51) (end 63.4447 51) (width 0.25) (layer F.Cu) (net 2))
 (segment (start 56.8146 53.7746) (end 54.4429 53.7746) (width 0.25) (layer F.Cu) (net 2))
 (segment (start 54.4429 53.7746) (end 53.5 54.7175) (width 0.25) (layer F.Cu) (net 2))
 (segment (start 53.5 54.7175) (end 53.5 54.8625) (width 0.25) (layer F.Cu) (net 2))
 (segment (start 58.04 55) (end 56.8146 53.7746) (width 0.25) (layer F.Cu) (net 2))
 (segment (start 58.1368 50.95) (end 56.8146 52.2722) (width 0.25) (layer F.Cu) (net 2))
 (segment (start 56.8146 52.2722) (end 56.8146 53.7746) (width 0.25) (layer F.Cu) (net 2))
 (segment (start 58.1368 50.95) (end 57.7247 50.95) (width 0.25) (layer F.Cu) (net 2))
 (segment (start 58.5 50.95) (end 58.1368 50.95) (width 0.25) (layer F.Cu) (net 2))
 (segment (start 54.55 48.9) (end 54.55 49.7553) (width 0.25) (layer F.Cu) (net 2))
 (segment (start 57.7247 50.95) (end 56.53 49.7553) (width 0.25) (layer F.Cu) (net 2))
 (segment (start 56.53 49.7553) (end 54.55 49.7553) (width 0.25) (layer F.Cu) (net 2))
 (segment (start 67 53.1375) (end 65.1553 51.2928) (width 0.25) (layer F.Cu) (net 2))
 (segment (start 65.1553 51.2928) (end 65.1553 51) (width 0.25) (layer F.Cu) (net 2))
 (segment (start 64.3 51) (end 65.1553 51) (width 0.25) (layer F.Cu) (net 2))
 (segment (start 53 56.85) (end 53 56.0747) (width 0.25) (layer F.Cu) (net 2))
 (segment (start 53 56.0747) (end 53.5 55.5747) (width 0.25) (layer F.Cu) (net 2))
 (segment (start 53.5 55.5747) (end 53.5 54.8625) (width 0.25) (layer F.Cu) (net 2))
 (segment (start 58.04 55) (end 58 55.04) (width 0.25) (layer F.Cu) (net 2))
 (segment (start 58 55.04) (end 58 58.1375) (width 0.25) (layer F.Cu) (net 2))
 (via (at 63.263 51.8396) (size 0.8) (layers F.Cu B.Cu) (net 2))
 (segment (start 62 58.0875) (end 61.96 58.0475) (width 0.25) (layer F.Cu) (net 3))
 (segment (start 61.96 58.0475) (end 61.96 55) (width 0.25) (layer F.Cu) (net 3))
 (segment (start 60.5 50.7253) (end 60.5 50.9349) (width 0.25) (layer F.Cu) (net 4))
 (segment (start 60.5 50.9349) (end 63.3398 53.7747) (width 0.25) (layer F.Cu) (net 4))
 (segment (start 63.3398 53.7747) (end 64.5 53.7747) (width 0.25) (layer F.Cu) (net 4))
 (segment (start 60.5 50) (end 60.5 50.7253) (width 0.25) (layer F.Cu) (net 4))
 (segment (start 64.5 55) (end 64.5 53.7747) (width 0.25) (layer F.Cu) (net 4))
 (segment (start 53 60.15) (end 53 60.9253) (width 0.25) (layer F.Cu) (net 5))
 (segment (start 56.75 63) (end 55.6647 63) (width 0.25) (layer F.Cu) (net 5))
 (segment (start 55.6647 63) (end 53.59 60.9253) (width 0.25) (layer F.Cu) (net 5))
 (segment (start 53.59 60.9253) (end 53 60.9253) (width 0.25) (layer F.Cu) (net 5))
 (segment (start 56.45 48.9) (end 56.45 48.0447) (width 0.25) (layer F.Cu) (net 6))
 (segment (start 57.5875 47) (end 56.5428 48.0447) (width 0.25) (layer F.Cu) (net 6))
 (segment (start 56.5428 48.0447) (end 56.45 48.0447) (width 0.25) (layer F.Cu) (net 6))
 (segment (start 55.5 51.9553) (end 53.274 51.9553) (width 0.25) (layer F.Cu) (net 7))
 (segment (start 53.274 51.9553) (end 51.6223 53.607) (width 0.25) (layer F.Cu) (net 7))
 (segment (start 51.6223 53.607) (end 51.6223 60.3354) (width 0.25) (layer F.Cu) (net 7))
 (segment (start 51.6223 60.3354) (end 55.3872 64.1003) (width 0.25) (layer F.Cu) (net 7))
 (segment (start 55.3872 64.1003) (end 59.1203 64.1003) (width 0.25) (layer F.Cu) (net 7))
 (segment (start 59.1203 64.1003) (end 60.56 65.54) (width 0.25) (layer F.Cu) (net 7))
 (segment (start 55.5 51.1) (end 55.5 51.9553) (width 0.25) (layer F.Cu) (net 7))
 (segment (start 62.5 49.0875) (end 61.6525 49.935) (width 0.25) (layer F.Cu) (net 10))
 (segment (start 61.6525 49.935) (end 61.6525 51.3564) (width 0.25) (layer F.Cu) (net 10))
 (segment (start 61.6525 51.3564) (end 63.0961 52.8) (width 0.25) (layer F.Cu) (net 10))
 (segment (start 63.0961 52.8) (end 64.6324 52.8) (width 0.25) (layer F.Cu) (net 10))
 (segment (start 64.6324 52.8) (end 65.7574 53.925) (width 0.25) (layer F.Cu) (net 10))
 (segment (start 65.7574 53.925) (end 65.7574 56.9673) (width 0.25) (layer F.Cu) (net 10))
 (segment (start 65.7574 56.9673) (end 65.5 57.2247) (width 0.25) (layer F.Cu) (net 10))
 (segment (start 65.5 58) (end 65.5 57.2247) (width 0.25) (layer F.Cu) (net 10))
 (segment (start 62.5 49.0875) (end 63.4625 50.05) (width 0.25) (layer F.Cu) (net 10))
 (segment (start 63.4625 50.05) (end 65.6447 50.05) (width 0.25) (layer F.Cu) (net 10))
 (segment (start 66.5 50.05) (end 65.6447 50.05) (width 0.25) (layer F.Cu) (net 10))
 (segment (start 64.3 49.1) (end 65.1553 49.1) (width 0.25) (layer F.Cu) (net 11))
 (segment (start 61.83 63) (end 64.771 63) (width 0.25) (layer F.Cu) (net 11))
 (segment (start 64.771 63) (end 68.2807 59.4903) (width 0.25) (layer F.Cu) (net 11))
 (segment (start 68.2807 59.4903) (end 68.2807 49.5363) (width 0.25) (layer F.Cu) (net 11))
 (segment (start 68.2807 49.5363) (end 67.1941 48.4497) (width 0.25) (layer F.Cu) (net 11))
 (segment (start 67.1941 48.4497) (end 65.8056 48.4497) (width 0.25) (layer F.Cu) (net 11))
 (segment (start 65.8056 48.4497) (end 65.1553 49.1) (width 0.25) (layer F.Cu) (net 11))
 (segment (start 63.8247 60) (end 63.0984 60.7263) (width 0.25) (layer F.Cu) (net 14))
 (segment (start 63.0984 60.7263) (end 54.983 60.7263) (width 0.25) (layer F.Cu) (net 14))
 (segment (start 54.983 60.7263) (end 54.6621 60.4054) (width 0.25) (layer F.Cu) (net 14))
 (segment (start 54.6621 60.4054) (end 54.6621 58.9254) (width 0.25) (layer F.Cu) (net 14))
 (segment (start 54.6621 58.9254) (end 55.5 58.0875) (width 0.25) (layer F.Cu) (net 14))
 (segment (start 64.55 60) (end 63.8247 60) (width 0.25) (layer F.Cu) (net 14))
 (segment (start 55.5 55) (end 55.5 58.0875) (width 0.25) (layer F.Cu) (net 14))
 (segment (start 58.5 49.05) (end 58.5 48.3247) (width 0.25) (layer F.Cu) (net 15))
 (segment (start 58.5 48.3247) (end 59.4125 47.4122) (width 0.25) (layer F.Cu) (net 15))
 (segment (start 59.4125 47.4122) (end 59.4125 47) (width 0.25) (layer F.Cu) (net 15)))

